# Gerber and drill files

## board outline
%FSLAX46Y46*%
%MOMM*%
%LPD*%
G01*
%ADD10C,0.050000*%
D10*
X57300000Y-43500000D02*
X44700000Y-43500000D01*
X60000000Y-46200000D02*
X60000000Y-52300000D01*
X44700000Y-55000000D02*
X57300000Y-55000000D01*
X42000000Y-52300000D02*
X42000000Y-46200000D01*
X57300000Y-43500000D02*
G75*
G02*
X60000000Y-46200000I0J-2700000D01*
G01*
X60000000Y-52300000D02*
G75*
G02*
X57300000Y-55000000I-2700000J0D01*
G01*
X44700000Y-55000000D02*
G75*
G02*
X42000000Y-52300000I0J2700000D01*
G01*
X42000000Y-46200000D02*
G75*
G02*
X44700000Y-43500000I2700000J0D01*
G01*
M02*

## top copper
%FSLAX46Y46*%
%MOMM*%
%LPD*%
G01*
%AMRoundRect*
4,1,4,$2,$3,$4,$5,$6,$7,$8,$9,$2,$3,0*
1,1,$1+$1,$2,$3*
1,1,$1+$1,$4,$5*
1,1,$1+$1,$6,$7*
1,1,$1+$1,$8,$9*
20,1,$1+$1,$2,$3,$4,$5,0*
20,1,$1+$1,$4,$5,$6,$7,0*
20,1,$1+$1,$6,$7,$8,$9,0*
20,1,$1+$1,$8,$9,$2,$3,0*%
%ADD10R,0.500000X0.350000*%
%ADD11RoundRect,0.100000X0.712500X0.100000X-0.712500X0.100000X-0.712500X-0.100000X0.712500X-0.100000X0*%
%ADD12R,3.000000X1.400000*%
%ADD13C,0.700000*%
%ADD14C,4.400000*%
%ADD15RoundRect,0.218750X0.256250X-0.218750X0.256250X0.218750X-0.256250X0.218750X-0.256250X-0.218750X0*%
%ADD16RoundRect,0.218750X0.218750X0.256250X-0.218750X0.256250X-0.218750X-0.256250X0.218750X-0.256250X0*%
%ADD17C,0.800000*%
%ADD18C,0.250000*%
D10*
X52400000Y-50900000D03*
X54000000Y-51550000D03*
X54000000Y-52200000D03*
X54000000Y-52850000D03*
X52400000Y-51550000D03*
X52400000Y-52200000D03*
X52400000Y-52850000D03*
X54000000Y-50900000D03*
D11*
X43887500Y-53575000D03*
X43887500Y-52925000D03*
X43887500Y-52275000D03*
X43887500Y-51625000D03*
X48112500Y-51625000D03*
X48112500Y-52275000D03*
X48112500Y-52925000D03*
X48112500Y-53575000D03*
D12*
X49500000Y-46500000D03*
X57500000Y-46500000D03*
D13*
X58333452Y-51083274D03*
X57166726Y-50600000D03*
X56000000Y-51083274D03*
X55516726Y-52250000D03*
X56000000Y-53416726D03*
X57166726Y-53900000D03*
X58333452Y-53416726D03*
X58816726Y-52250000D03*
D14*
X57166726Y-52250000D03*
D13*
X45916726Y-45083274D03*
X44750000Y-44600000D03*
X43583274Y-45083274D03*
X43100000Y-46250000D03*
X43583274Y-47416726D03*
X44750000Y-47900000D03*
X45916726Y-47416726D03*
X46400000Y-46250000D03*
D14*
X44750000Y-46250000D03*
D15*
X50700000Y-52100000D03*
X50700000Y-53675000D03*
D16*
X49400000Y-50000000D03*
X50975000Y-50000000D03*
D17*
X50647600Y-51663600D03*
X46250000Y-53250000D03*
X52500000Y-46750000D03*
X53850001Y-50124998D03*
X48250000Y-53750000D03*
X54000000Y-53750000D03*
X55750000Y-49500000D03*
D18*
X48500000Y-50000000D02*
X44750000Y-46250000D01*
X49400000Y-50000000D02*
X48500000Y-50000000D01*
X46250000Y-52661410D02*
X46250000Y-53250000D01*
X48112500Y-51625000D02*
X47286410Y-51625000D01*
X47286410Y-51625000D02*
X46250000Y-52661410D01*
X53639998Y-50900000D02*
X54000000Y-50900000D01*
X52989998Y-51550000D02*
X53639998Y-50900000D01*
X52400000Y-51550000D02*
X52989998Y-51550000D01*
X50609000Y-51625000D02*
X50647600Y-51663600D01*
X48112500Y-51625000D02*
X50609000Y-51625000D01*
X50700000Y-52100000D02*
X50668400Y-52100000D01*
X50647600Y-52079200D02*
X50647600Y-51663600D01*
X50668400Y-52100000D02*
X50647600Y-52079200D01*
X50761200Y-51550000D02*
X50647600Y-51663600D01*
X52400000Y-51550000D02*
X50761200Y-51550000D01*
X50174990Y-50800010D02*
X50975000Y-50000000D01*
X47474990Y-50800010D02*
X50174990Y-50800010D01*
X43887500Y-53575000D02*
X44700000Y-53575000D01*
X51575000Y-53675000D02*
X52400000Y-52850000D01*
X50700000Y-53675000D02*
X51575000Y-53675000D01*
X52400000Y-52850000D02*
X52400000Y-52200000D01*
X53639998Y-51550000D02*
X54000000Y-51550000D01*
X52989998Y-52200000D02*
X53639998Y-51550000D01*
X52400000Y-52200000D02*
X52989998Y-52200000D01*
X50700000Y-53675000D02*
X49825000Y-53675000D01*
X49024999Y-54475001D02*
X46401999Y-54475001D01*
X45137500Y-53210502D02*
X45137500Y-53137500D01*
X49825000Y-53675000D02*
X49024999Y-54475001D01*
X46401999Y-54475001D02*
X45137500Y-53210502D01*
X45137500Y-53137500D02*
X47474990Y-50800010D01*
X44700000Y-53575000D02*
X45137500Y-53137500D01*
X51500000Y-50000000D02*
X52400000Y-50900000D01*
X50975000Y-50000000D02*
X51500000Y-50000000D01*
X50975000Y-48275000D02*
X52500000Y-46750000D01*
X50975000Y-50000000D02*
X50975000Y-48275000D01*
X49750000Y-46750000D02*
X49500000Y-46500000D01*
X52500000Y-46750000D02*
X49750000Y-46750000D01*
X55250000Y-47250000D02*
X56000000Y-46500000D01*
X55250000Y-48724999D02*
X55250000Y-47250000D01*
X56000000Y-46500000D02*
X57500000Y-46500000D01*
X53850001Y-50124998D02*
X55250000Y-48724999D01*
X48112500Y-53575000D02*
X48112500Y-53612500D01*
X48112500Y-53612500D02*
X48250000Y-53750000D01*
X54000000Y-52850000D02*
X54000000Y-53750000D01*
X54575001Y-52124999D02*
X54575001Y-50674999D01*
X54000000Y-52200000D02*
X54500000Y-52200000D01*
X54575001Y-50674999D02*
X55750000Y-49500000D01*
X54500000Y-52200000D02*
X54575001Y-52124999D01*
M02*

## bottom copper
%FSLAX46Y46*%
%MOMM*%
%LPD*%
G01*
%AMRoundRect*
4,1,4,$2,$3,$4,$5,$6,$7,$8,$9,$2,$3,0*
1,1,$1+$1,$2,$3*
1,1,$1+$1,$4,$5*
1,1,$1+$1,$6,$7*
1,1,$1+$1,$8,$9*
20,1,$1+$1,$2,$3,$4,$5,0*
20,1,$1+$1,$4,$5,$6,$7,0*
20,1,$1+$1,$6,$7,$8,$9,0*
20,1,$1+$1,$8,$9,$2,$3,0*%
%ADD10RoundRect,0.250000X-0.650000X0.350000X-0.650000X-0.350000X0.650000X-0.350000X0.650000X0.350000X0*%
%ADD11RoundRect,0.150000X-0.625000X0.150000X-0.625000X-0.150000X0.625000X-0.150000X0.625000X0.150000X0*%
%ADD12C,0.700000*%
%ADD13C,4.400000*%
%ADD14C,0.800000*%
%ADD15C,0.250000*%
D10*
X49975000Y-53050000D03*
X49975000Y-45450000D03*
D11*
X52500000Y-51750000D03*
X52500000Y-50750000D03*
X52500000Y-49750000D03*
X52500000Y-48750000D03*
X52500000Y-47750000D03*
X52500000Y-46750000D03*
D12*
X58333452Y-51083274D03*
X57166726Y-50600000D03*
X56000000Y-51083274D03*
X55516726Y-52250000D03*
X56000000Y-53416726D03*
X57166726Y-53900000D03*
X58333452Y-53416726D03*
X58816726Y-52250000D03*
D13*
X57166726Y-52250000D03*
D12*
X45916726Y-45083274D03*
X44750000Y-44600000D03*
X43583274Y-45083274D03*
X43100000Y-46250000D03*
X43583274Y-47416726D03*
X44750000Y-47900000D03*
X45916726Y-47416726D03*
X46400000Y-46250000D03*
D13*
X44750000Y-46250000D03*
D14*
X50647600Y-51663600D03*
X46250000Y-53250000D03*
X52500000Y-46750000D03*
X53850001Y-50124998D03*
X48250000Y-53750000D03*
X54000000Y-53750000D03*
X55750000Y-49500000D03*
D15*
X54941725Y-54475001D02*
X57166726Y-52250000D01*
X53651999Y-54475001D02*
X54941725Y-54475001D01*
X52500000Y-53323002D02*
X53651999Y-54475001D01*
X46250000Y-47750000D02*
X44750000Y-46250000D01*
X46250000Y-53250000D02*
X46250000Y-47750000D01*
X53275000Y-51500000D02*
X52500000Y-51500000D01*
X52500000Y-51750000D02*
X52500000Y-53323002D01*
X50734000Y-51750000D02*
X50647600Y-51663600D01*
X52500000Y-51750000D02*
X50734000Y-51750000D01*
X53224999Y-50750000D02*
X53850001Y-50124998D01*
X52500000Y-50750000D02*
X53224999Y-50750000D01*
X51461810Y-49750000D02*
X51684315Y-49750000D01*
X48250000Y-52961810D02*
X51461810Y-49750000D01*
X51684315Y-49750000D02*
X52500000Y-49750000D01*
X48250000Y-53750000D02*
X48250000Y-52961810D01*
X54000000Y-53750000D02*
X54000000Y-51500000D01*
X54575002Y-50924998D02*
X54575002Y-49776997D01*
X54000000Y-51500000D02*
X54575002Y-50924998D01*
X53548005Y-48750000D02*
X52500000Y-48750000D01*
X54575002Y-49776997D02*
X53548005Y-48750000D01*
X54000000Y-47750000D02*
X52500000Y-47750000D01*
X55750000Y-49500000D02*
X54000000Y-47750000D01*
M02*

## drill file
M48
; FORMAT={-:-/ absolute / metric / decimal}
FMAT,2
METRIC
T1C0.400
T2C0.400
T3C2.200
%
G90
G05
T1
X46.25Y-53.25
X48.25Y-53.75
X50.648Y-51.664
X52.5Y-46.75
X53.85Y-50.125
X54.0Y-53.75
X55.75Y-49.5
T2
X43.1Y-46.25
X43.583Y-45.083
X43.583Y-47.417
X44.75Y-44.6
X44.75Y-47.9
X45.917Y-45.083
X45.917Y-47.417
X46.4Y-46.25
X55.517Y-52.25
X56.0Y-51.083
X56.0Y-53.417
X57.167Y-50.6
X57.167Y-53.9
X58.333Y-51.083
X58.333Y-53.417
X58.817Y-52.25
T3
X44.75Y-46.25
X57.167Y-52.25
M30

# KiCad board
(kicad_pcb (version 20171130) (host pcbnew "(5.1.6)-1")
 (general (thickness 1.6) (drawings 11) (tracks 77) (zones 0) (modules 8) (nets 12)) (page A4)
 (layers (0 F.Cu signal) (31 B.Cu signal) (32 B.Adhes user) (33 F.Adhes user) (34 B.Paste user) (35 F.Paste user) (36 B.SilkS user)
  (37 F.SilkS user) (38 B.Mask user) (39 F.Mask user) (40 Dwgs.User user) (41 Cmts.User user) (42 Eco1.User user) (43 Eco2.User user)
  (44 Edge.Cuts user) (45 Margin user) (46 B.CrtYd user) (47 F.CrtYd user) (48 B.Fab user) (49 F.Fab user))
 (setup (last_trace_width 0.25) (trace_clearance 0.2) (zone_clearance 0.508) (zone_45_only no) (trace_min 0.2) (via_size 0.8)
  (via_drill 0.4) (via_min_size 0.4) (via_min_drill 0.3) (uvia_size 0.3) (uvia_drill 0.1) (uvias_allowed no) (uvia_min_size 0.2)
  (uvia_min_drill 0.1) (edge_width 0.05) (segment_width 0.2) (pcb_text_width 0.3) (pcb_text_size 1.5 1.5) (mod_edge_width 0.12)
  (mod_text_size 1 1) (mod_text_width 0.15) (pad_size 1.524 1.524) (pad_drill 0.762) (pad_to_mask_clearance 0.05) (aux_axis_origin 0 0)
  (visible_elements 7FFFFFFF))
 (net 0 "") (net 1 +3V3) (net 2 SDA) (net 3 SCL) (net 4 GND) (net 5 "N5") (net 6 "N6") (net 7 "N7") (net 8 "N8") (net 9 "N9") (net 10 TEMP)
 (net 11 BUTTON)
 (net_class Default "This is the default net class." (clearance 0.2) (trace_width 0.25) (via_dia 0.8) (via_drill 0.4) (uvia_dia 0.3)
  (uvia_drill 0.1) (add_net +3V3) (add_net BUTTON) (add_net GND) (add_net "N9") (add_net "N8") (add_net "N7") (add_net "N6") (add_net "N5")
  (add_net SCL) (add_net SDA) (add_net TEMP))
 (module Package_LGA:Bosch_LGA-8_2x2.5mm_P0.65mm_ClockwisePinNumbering (layer F.Cu) (at 53.2 51.875 270)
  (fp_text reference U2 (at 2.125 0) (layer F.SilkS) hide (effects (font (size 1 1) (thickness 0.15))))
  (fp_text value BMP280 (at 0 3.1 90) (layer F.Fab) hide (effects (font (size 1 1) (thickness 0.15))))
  (pad 8 smd rect (at -0.975 0.8) (size 0.5 0.35) (layers F.Cu F.Paste F.Mask) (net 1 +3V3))
  (pad 2 smd rect (at -0.325 -0.8) (size 0.5 0.35) (layers F.Cu F.Paste F.Mask) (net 1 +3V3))
  (pad 3 smd rect (at 0.325 -0.8) (size 0.5 0.35) (layers F.Cu F.Paste F.Mask) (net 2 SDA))
  (pad 4 smd rect (at 0.975 -0.8) (size 0.5 0.35) (layers F.Cu F.Paste F.Mask) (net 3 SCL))
  (pad 7 smd rect (at -0.325 0.8) (size 0.5 0.35) (layers F.Cu F.Paste F.Mask) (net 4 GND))
  (pad 6 smd rect (at 0.325 0.8) (size 0.5 0.35) (layers F.Cu F.Paste F.Mask) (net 1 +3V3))
  (pad 5 smd rect (at 0.975 0.8) (size 0.5 0.35) (layers F.Cu F.Paste F.Mask) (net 1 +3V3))
  (pad 1 smd rect (at -0.975 -0.8) (size 0.5 0.35) (layers F.Cu F.Paste F.Mask) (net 4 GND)))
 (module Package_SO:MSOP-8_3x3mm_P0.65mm (layer F.Cu) (at 46 52.6 180)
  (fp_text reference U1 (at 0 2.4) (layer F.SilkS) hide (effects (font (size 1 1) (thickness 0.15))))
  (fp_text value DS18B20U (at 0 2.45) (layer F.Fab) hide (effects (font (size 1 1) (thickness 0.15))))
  (pad 8 smd roundrect (at 2.1125 -0.975 180) (size 1.625 0.4) (layers F.Cu F.Paste F.Mask) (roundrect_rratio 0.25) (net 1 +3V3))
  (pad 7 smd roundrect (at 2.1125 -0.325 180) (size 1.625 0.4) (layers F.Cu F.Paste F.Mask) (roundrect_rratio 0.25) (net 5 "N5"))
  (pad 6 smd roundrect (at 2.1125 0.325 180) (size 1.625 0.4) (layers F.Cu F.Paste F.Mask) (roundrect_rratio 0.25) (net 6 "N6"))
  (pad 5 smd roundrect (at 2.1125 0.975 180) (size 1.625 0.4) (layers F.Cu F.Paste F.Mask) (roundrect_rratio 0.25) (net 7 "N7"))
  (pad 4 smd roundrect (at -2.1125 0.975 180) (size 1.625 0.4) (layers F.Cu F.Paste F.Mask) (roundrect_rratio 0.25) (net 4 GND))
  (pad 3 smd roundrect (at -2.1125 0.325 180) (size 1.625 0.4) (layers F.Cu F.Paste F.Mask) (roundrect_rratio 0.25) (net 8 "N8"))
  (pad 2 smd roundrect (at -2.1125 -0.325 180) (size 1.625 0.4) (layers F.Cu F.Paste F.Mask) (roundrect_rratio 0.25) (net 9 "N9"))
  (pad 1 smd roundrect (at -2.1125 -0.975 180) (size 1.625 0.4) (layers F.Cu F.Paste F.Mask) (roundrect_rratio 0.25) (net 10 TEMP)))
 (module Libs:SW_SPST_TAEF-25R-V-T (layer F.Cu) (at 53.5 46.5)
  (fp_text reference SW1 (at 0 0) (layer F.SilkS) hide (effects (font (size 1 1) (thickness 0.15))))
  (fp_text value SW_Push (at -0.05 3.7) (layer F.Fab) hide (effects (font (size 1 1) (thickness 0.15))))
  (pad 1 smd rect (at -4 0) (size 3 1.4) (layers F.Cu F.Paste F.Mask) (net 1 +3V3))
  (pad 2 smd rect (at 4 0) (size 3 1.4) (layers F.Cu F.Paste F.Mask) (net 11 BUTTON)))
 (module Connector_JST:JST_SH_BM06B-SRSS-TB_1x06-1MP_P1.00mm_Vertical (layer B.Cu) (at 51.175 49.25 270)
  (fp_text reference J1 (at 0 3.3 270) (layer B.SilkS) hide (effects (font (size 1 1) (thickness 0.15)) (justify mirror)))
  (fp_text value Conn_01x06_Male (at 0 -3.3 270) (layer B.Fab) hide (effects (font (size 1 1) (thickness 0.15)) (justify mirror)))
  (pad MP smd roundrect (at 3.8 1.2 270) (size 1.2 1.8) (layers B.Cu B.Paste B.Mask) (roundrect_rratio 0.208333))
  (pad MP smd roundrect (at -3.8 1.2 270) (size 1.2 1.8) (layers B.Cu B.Paste B.Mask) (roundrect_rratio 0.208333))
  (pad 6 smd roundrect (at 2.5 -1.325 270) (size 0.6 1.55) (layers B.Cu B.Paste B.Mask) (roundrect_rratio 0.25) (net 4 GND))
  (pad 5 smd roundrect (at 1.5 -1.325 270) (size 0.6 1.55) (layers B.Cu B.Paste B.Mask) (roundrect_rratio 0.25) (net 11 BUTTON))
  (pad 4 smd roundrect (at 0.5 -1.325 270) (size 0.6 1.55) (layers B.Cu B.Paste B.Mask) (roundrect_rratio 0.25) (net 10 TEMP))
  (pad 3 smd roundrect (at -0.5 -1.325 270) (size 0.6 1.55) (layers B.Cu B.Paste B.Mask) (roundrect_rratio 0.25) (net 3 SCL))
  (pad 2 smd roundrect (at -1.5 -1.325 270) (size 0.6 1.55) (layers B.Cu B.Paste B.Mask) (roundrect_rratio 0.25) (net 2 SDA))
  (pad 1 smd roundrect (at -2.5 -1.325 270) (size 0.6 1.55) (layers B.Cu B.Paste B.Mask) (roundrect_rratio 0.25) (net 1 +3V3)))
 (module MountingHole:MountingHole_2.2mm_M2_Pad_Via (layer F.Cu) (at 57.166726 52.25)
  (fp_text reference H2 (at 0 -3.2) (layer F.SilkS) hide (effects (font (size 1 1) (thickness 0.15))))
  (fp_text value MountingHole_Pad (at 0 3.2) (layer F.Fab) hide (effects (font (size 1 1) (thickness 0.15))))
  (pad 1 thru_hole circle (at 1.166726 -1.166726) (size 0.7 0.7) (drill 0.4) (layers *.Cu *.Mask) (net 4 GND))
  (pad 1 thru_hole circle (at 0 -1.65) (size 0.7 0.7) (drill 0.4) (layers *.Cu *.Mask) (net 4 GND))
  (pad 1 thru_hole circle (at -1.166726 -1.166726) (size 0.7 0.7) (drill 0.4) (layers *.Cu *.Mask) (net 4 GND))
  (pad 1 thru_hole circle (at -1.65 0) (size 0.7 0.7) (drill 0.4) (layers *.Cu *.Mask) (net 4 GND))
  (pad 1 thru_hole circle (at -1.166726 1.166726) (size 0.7 0.7) (drill 0.4) (layers *.Cu *.Mask) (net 4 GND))
  (pad 1 thru_hole circle (at 0 1.65) (size 0.7 0.7) (drill 0.4) (layers *.Cu *.Mask) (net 4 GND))
  (pad 1 thru_hole circle (at 1.166726 1.166726) (size 0.7 0.7) (drill 0.4) (layers *.Cu *.Mask) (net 4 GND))
  (pad 1 thru_hole circle (at 1.65 0) (size 0.7 0.7) (drill 0.4) (layers *.Cu *.Mask) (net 4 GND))
  (pad 1 thru_hole circle (at 0 0) (size 4.4 4.4) (drill 2.2) (layers *.Cu *.Mask) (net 4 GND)))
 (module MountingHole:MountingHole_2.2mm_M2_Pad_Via (layer F.Cu) (at 44.75 46.25)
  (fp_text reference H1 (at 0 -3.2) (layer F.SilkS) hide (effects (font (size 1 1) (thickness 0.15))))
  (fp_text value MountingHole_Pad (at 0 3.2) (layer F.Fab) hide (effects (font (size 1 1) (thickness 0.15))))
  (pad 1 thru_hole circle (at 1.166726 -1.166726) (size 0.7 0.7) (drill 0.4) (layers *.Cu *.Mask) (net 4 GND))
  (pad 1 thru_hole circle (at 0 -1.65) (size 0.7 0.7) (drill 0.4) (layers *.Cu *.Mask) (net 4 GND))
  (pad 1 thru_hole circle (at -1.166726 -1.166726) (size 0.7 0.7) (drill 0.4) (layers *.Cu *.Mask) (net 4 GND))
  (pad 1 thru_hole circle (at -1.65 0) (size 0.7 0.7) (drill 0.4) (layers *.Cu *.Mask) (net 4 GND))
  (pad 1 thru_hole circle (at -1.166726 1.166726) (size 0.7 0.7) (drill 0.4) (layers *.Cu *.Mask) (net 4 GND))
  (pad 1 thru_hole circle (at 0 1.65) (size 0.7 0.7) (drill 0.4) (layers *.Cu *.Mask) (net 4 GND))
  (pad 1 thru_hole circle (at 1.166726 1.166726) (size 0.7 0.7) (drill 0.4) (layers *.Cu *.Mask) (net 4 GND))
  (pad 1 thru_hole circle (at 1.65 0) (size 0.7 0.7) (drill 0.4) (layers *.Cu *.Mask) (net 4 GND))
  (pad 1 thru_hole circle (at 0 0) (size 4.4 4.4) (drill 2.2) (layers *.Cu *.Mask) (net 4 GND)))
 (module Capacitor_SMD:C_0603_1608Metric (layer F.Cu) (at 50.7 52.8875 90)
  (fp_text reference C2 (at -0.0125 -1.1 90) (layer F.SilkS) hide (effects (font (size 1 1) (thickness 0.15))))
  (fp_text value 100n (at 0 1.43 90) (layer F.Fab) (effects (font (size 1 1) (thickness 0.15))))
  (pad 2 smd roundrect (at 0.7875 0 90) (size 0.875 0.95) (layers F.Cu F.Paste F.Mask) (roundrect_rratio 0.25) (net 4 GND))
  (pad 1 smd roundrect (at -0.7875 0 90) (size 0.875 0.95) (layers F.Cu F.Paste F.Mask) (roundrect_rratio 0.25) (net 1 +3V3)))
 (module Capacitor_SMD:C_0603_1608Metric (layer F.Cu) (at 50.1875 50 180)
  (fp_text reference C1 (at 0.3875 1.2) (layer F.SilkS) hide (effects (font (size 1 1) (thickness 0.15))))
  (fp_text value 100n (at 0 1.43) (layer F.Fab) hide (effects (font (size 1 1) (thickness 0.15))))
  (pad 2 smd roundrect (at 0.7875 0 180) (size 0.875 0.95) (layers F.Cu F.Paste F.Mask) (roundrect_rratio 0.25) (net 4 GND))
  (pad 1 smd roundrect (at -0.7875 0 180) (size 0.875 0.95) (layers F.Cu F.Paste F.Mask) (roundrect_rratio 0.25) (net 1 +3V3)))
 (gr_line (start 57.3 43.5) (end 44.7 43.5) (layer Edge.Cuts) (width 0.05))
 (gr_line (start 60 46.2) (end 60 52.3) (layer Edge.Cuts) (width 0.05))
 (gr_line (start 44.7 55) (end 57.3 55) (layer Edge.Cuts) (width 0.05))
 (gr_line (start 42 52.3) (end 42 46.2) (layer Edge.Cuts) (width 0.05))
 (gr_arc (start 57.3 46.2) (end 60 46.2) (angle -90) (layer Edge.Cuts) (width 0.05))
 (gr_arc (start 57.3 52.3) (end 57.3 55) (angle -90) (layer Edge.Cuts) (width 0.05))
 (gr_arc (start 44.7 52.3) (end 42 52.3) (angle -90) (layer Edge.Cuts) (width 0.05))
 (gr_arc (start 44.7 46.2) (end 44.7 43.5) (angle -90) (layer Edge.Cuts) (width 0.05))
 (via (at 50.6476 51.6636) (size 0.8) (drill 0.4) (layers F.Cu B.Cu) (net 4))
 (segment (start 54.941725 54.475001) (end 57.166726 52.25) (width 0.25) (layer B.Cu) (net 4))
 (segment (start 53.651999 54.475001) (end 54.941725 54.475001) (width 0.25) (layer B.Cu) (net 4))
 (segment (start 52.5 53.323002) (end 53.651999 54.475001) (width 0.25) (layer B.Cu) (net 4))
 (segment (start 48.5 50) (end 44.75 46.25) (width 0.25) (layer F.Cu) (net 4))
 (segment (start 49.4 50) (end 48.5 50) (width 0.25) (layer F.Cu) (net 4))
 (via (at 46.25 53.25) (size 0.8) (drill 0.4) (layers F.Cu B.Cu) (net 4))
 (segment (start 46.25 52.66141) (end 46.25 53.25) (width 0.25) (layer F.Cu) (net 4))
 (segment (start 48.1125 51.625) (end 47.28641 51.625) (width 0.25) (layer F.Cu) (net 4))
 (segment (start 47.28641 51.625) (end 46.25 52.66141) (width 0.25) (layer F.Cu) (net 4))
 (segment (start 46.25 47.75) (end 44.75 46.25) (width 0.25) (layer B.Cu) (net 4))
 (segment (start 46.25 53.25) (end 46.25 47.75) (width 0.25) (layer B.Cu) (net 4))
 (segment (start 53.639998 50.9) (end 54 50.9) (width 0.25) (layer F.Cu) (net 4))
 (segment (start 52.989998 51.55) (end 53.639998 50.9) (width 0.25) (layer F.Cu) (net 4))
 (segment (start 52.4 51.55) (end 52.989998 51.55) (width 0.25) (layer F.Cu) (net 4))
 (segment (start 53.275 51.5) (end 52.5 51.5) (width 0.25) (layer B.Cu) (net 4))
 (segment (start 52.5 51.75) (end 52.5 53.323002) (width 0.25) (layer B.Cu) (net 4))
 (segment (start 50.734 51.75) (end 50.6476 51.6636) (width 0.25) (layer B.Cu) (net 4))
 (segment (start 52.5 51.75) (end 50.734 51.75) (width 0.25) (layer B.Cu) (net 4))
 (segment (start 50.609 51.625) (end 50.6476 51.6636) (width 0.25) (layer F.Cu) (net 4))
 (segment (start 48.1125 51.625) (end 50.609 51.625) (width 0.25) (layer F.Cu) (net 4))
 (segment (start 50.7 52.1) (end 50.6684 52.1) (width 0.25) (layer F.Cu) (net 4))
 (segment (start 50.6476 52.0792) (end 50.6476 51.6636) (width 0.25) (layer F.Cu) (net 4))
 (segment (start 50.6684 52.1) (end 50.6476 52.0792) (width 0.25) (layer F.Cu) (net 4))
 (segment (start 50.7612 51.55) (end 50.6476 51.6636) (width 0.25) (layer F.Cu) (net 4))
 (segment (start 52.4 51.55) (end 50.7612 51.55) (width 0.25) (layer F.Cu) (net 4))
 (segment (start 50.17499 50.80001) (end 50.975 50) (width 0.25) (layer F.Cu) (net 1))
 (segment (start 47.47499 50.80001) (end 50.17499 50.80001) (width 0.25) (layer F.Cu) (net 1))
 (segment (start 43.8875 53.575) (end 44.7 53.575) (width 0.25) (layer F.Cu) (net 1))
 (segment (start 51.575 53.675) (end 52.4 52.85) (width 0.25) (layer F.Cu) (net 1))
 (segment (start 50.7 53.675) (end 51.575 53.675) (width 0.25) (layer F.Cu) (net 1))
 (segment (start 52.4 52.85) (end 52.4 52.2) (width 0.25) (layer F.Cu) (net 1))
 (segment (start 53.639998 51.55) (end 54 51.55) (width 0.25) (layer F.Cu) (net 1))
 (segment (start 52.989998 52.2) (end 53.639998 51.55) (width 0.25) (layer F.Cu) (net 1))
 (segment (start 52.4 52.2) (end 52.989998 52.2) (width 0.25) (layer F.Cu) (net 1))
 (segment (start 50.7 53.675) (end 49.825 53.675) (width 0.25) (layer F.Cu) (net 1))
 (segment (start 49.024999 54.475001) (end 46.401999 54.475001) (width 0.25) (layer F.Cu) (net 1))
 (segment (start 45.1375 53.210502) (end 45.1375 53.1375) (width 0.25) (layer F.Cu) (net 1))
 (segment (start 49.825 53.675) (end 49.024999 54.475001) (width 0.25) (layer F.Cu) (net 1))
 (segment (start 46.401999 54.475001) (end 45.1375 53.210502) (width 0.25) (layer F.Cu) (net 1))
 (segment (start 45.1375 53.1375) (end 47.47499 50.80001) (width 0.25) (layer F.Cu) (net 1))
 (segment (start 44.7 53.575) (end 45.1375 53.1375) (width 0.25) (layer F.Cu) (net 1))
 (segment (start 51.5 50) (end 52.4 50.9) (width 0.25) (layer F.Cu) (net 1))
 (segment (start 50.975 50) (end 51.5 50) (width 0.25) (layer F.Cu) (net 1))
 (via (at 52.5 46.75) (size 0.8) (drill 0.4) (layers F.Cu B.Cu) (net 1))
 (segment (start 50.975 48.275) (end 52.5 46.75) (width 0.25) (layer F.Cu) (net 1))
 (segment (start 50.975 50) (end 50.975 48.275) (width 0.25) (layer F.Cu) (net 1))
 (segment (start 49.75 46.75) (end 49.5 46.5) (width 0.25) (layer F.Cu) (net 1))
 (segment (start 52.5 46.75) (end 49.75 46.75) (width 0.25) (layer F.Cu) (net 1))
 (segment (start 55.25 47.25) (end 56 46.5) (width 0.25) (layer F.Cu) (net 11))
 (segment (start 55.25 48.724999) (end 55.25 47.25) (width 0.25) (layer F.Cu) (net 11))
 (via (at 53.850001 50.124998) (size 0.8) (drill 0.4) (layers F.Cu B.Cu) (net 11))
 (segment (start 56 46.5) (end 57.5 46.5) (width 0.25) (layer F.Cu) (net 11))
 (segment (start 53.850001 50.124998) (end 55.25 48.724999) (width 0.25) (layer F.Cu) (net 11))
 (segment (start 53.224999 50.75) (end 53.850001 50.124998) (width 0.25) (layer B.Cu) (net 11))
 (segment (start 52.5 50.75) (end 53.224999 50.75) (width 0.25) (layer B.Cu) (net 11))
 (via (at 48.25 53.75) (size 0.8) (drill 0.4) (layers F.Cu B.Cu) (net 10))
 (segment (start 48.1125 53.575) (end 48.1125 53.6125) (width 0.25) (layer F.Cu) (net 10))
 (segment (start 48.1125 53.6125) (end 48.25 53.75) (width 0.25) (layer F.Cu) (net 10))
 (segment (start 51.46181 49.75) (end 51.684315 49.75) (width 0.25) (layer B.Cu) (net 10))
 (segment (start 48.25 52.96181) (end 51.46181 49.75) (width 0.25) (layer B.Cu) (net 10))
 (segment (start 51.684315 49.75) (end 52.5 49.75) (width 0.25) (layer B.Cu) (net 10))
 (segment (start 48.25 53.75) (end 48.25 52.96181) (width 0.25) (layer B.Cu) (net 10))
 (via (at 54 53.75) (size 0.8) (drill 0.4) (layers F.Cu B.Cu) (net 3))
 (segment (start 54 52.85) (end 54 53.75) (width 0.25) (layer F.Cu) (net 3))
 (segment (start 54 53.75) (end 54 51.5) (width 0.25) (layer B.Cu) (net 3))
 (segment (start 54.575002 50.924998) (end 54.575002 49.776997) (width 0.25) (layer B.Cu) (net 3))
 (segment (start 54 51.5) (end 54.575002 50.924998) (width 0.25) (layer B.Cu) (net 3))
 (segment (start 53.548005 48.75) (end 52.5 48.75) (width 0.25) (layer B.Cu) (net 3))
 (segment (start 54.575002 49.776997) (end 53.548005 48.75) (width 0.25) (layer B.Cu) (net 3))
 (segment (start 54.575001 52.124999) (end 54.575001 50.674999) (width 0.25) (layer F.Cu) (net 2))
 (via (at 55.75 49.5) (size 0.8) (drill 0.4) (layers F.Cu B.Cu) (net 2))
 (segment (start 54 52.2) (end 54.5 52.2) (width 0.25) (layer F.Cu) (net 2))
 (segment (start 54.575001 50.674999) (end 55.75 49.5) (width 0.25) (layer F.Cu) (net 2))
 (segment (start 54.5 52.2) (end 54.575001 52.124999) (width 0.25) (layer F.Cu) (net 2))
 (segment (start 54 47.75) (end 52.5 47.75) (width 0.25) (layer B.Cu) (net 2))
 (segment (start 55.75 49.5) (end 54 47.75) (width 0.25) (layer B.Cu) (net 2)))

